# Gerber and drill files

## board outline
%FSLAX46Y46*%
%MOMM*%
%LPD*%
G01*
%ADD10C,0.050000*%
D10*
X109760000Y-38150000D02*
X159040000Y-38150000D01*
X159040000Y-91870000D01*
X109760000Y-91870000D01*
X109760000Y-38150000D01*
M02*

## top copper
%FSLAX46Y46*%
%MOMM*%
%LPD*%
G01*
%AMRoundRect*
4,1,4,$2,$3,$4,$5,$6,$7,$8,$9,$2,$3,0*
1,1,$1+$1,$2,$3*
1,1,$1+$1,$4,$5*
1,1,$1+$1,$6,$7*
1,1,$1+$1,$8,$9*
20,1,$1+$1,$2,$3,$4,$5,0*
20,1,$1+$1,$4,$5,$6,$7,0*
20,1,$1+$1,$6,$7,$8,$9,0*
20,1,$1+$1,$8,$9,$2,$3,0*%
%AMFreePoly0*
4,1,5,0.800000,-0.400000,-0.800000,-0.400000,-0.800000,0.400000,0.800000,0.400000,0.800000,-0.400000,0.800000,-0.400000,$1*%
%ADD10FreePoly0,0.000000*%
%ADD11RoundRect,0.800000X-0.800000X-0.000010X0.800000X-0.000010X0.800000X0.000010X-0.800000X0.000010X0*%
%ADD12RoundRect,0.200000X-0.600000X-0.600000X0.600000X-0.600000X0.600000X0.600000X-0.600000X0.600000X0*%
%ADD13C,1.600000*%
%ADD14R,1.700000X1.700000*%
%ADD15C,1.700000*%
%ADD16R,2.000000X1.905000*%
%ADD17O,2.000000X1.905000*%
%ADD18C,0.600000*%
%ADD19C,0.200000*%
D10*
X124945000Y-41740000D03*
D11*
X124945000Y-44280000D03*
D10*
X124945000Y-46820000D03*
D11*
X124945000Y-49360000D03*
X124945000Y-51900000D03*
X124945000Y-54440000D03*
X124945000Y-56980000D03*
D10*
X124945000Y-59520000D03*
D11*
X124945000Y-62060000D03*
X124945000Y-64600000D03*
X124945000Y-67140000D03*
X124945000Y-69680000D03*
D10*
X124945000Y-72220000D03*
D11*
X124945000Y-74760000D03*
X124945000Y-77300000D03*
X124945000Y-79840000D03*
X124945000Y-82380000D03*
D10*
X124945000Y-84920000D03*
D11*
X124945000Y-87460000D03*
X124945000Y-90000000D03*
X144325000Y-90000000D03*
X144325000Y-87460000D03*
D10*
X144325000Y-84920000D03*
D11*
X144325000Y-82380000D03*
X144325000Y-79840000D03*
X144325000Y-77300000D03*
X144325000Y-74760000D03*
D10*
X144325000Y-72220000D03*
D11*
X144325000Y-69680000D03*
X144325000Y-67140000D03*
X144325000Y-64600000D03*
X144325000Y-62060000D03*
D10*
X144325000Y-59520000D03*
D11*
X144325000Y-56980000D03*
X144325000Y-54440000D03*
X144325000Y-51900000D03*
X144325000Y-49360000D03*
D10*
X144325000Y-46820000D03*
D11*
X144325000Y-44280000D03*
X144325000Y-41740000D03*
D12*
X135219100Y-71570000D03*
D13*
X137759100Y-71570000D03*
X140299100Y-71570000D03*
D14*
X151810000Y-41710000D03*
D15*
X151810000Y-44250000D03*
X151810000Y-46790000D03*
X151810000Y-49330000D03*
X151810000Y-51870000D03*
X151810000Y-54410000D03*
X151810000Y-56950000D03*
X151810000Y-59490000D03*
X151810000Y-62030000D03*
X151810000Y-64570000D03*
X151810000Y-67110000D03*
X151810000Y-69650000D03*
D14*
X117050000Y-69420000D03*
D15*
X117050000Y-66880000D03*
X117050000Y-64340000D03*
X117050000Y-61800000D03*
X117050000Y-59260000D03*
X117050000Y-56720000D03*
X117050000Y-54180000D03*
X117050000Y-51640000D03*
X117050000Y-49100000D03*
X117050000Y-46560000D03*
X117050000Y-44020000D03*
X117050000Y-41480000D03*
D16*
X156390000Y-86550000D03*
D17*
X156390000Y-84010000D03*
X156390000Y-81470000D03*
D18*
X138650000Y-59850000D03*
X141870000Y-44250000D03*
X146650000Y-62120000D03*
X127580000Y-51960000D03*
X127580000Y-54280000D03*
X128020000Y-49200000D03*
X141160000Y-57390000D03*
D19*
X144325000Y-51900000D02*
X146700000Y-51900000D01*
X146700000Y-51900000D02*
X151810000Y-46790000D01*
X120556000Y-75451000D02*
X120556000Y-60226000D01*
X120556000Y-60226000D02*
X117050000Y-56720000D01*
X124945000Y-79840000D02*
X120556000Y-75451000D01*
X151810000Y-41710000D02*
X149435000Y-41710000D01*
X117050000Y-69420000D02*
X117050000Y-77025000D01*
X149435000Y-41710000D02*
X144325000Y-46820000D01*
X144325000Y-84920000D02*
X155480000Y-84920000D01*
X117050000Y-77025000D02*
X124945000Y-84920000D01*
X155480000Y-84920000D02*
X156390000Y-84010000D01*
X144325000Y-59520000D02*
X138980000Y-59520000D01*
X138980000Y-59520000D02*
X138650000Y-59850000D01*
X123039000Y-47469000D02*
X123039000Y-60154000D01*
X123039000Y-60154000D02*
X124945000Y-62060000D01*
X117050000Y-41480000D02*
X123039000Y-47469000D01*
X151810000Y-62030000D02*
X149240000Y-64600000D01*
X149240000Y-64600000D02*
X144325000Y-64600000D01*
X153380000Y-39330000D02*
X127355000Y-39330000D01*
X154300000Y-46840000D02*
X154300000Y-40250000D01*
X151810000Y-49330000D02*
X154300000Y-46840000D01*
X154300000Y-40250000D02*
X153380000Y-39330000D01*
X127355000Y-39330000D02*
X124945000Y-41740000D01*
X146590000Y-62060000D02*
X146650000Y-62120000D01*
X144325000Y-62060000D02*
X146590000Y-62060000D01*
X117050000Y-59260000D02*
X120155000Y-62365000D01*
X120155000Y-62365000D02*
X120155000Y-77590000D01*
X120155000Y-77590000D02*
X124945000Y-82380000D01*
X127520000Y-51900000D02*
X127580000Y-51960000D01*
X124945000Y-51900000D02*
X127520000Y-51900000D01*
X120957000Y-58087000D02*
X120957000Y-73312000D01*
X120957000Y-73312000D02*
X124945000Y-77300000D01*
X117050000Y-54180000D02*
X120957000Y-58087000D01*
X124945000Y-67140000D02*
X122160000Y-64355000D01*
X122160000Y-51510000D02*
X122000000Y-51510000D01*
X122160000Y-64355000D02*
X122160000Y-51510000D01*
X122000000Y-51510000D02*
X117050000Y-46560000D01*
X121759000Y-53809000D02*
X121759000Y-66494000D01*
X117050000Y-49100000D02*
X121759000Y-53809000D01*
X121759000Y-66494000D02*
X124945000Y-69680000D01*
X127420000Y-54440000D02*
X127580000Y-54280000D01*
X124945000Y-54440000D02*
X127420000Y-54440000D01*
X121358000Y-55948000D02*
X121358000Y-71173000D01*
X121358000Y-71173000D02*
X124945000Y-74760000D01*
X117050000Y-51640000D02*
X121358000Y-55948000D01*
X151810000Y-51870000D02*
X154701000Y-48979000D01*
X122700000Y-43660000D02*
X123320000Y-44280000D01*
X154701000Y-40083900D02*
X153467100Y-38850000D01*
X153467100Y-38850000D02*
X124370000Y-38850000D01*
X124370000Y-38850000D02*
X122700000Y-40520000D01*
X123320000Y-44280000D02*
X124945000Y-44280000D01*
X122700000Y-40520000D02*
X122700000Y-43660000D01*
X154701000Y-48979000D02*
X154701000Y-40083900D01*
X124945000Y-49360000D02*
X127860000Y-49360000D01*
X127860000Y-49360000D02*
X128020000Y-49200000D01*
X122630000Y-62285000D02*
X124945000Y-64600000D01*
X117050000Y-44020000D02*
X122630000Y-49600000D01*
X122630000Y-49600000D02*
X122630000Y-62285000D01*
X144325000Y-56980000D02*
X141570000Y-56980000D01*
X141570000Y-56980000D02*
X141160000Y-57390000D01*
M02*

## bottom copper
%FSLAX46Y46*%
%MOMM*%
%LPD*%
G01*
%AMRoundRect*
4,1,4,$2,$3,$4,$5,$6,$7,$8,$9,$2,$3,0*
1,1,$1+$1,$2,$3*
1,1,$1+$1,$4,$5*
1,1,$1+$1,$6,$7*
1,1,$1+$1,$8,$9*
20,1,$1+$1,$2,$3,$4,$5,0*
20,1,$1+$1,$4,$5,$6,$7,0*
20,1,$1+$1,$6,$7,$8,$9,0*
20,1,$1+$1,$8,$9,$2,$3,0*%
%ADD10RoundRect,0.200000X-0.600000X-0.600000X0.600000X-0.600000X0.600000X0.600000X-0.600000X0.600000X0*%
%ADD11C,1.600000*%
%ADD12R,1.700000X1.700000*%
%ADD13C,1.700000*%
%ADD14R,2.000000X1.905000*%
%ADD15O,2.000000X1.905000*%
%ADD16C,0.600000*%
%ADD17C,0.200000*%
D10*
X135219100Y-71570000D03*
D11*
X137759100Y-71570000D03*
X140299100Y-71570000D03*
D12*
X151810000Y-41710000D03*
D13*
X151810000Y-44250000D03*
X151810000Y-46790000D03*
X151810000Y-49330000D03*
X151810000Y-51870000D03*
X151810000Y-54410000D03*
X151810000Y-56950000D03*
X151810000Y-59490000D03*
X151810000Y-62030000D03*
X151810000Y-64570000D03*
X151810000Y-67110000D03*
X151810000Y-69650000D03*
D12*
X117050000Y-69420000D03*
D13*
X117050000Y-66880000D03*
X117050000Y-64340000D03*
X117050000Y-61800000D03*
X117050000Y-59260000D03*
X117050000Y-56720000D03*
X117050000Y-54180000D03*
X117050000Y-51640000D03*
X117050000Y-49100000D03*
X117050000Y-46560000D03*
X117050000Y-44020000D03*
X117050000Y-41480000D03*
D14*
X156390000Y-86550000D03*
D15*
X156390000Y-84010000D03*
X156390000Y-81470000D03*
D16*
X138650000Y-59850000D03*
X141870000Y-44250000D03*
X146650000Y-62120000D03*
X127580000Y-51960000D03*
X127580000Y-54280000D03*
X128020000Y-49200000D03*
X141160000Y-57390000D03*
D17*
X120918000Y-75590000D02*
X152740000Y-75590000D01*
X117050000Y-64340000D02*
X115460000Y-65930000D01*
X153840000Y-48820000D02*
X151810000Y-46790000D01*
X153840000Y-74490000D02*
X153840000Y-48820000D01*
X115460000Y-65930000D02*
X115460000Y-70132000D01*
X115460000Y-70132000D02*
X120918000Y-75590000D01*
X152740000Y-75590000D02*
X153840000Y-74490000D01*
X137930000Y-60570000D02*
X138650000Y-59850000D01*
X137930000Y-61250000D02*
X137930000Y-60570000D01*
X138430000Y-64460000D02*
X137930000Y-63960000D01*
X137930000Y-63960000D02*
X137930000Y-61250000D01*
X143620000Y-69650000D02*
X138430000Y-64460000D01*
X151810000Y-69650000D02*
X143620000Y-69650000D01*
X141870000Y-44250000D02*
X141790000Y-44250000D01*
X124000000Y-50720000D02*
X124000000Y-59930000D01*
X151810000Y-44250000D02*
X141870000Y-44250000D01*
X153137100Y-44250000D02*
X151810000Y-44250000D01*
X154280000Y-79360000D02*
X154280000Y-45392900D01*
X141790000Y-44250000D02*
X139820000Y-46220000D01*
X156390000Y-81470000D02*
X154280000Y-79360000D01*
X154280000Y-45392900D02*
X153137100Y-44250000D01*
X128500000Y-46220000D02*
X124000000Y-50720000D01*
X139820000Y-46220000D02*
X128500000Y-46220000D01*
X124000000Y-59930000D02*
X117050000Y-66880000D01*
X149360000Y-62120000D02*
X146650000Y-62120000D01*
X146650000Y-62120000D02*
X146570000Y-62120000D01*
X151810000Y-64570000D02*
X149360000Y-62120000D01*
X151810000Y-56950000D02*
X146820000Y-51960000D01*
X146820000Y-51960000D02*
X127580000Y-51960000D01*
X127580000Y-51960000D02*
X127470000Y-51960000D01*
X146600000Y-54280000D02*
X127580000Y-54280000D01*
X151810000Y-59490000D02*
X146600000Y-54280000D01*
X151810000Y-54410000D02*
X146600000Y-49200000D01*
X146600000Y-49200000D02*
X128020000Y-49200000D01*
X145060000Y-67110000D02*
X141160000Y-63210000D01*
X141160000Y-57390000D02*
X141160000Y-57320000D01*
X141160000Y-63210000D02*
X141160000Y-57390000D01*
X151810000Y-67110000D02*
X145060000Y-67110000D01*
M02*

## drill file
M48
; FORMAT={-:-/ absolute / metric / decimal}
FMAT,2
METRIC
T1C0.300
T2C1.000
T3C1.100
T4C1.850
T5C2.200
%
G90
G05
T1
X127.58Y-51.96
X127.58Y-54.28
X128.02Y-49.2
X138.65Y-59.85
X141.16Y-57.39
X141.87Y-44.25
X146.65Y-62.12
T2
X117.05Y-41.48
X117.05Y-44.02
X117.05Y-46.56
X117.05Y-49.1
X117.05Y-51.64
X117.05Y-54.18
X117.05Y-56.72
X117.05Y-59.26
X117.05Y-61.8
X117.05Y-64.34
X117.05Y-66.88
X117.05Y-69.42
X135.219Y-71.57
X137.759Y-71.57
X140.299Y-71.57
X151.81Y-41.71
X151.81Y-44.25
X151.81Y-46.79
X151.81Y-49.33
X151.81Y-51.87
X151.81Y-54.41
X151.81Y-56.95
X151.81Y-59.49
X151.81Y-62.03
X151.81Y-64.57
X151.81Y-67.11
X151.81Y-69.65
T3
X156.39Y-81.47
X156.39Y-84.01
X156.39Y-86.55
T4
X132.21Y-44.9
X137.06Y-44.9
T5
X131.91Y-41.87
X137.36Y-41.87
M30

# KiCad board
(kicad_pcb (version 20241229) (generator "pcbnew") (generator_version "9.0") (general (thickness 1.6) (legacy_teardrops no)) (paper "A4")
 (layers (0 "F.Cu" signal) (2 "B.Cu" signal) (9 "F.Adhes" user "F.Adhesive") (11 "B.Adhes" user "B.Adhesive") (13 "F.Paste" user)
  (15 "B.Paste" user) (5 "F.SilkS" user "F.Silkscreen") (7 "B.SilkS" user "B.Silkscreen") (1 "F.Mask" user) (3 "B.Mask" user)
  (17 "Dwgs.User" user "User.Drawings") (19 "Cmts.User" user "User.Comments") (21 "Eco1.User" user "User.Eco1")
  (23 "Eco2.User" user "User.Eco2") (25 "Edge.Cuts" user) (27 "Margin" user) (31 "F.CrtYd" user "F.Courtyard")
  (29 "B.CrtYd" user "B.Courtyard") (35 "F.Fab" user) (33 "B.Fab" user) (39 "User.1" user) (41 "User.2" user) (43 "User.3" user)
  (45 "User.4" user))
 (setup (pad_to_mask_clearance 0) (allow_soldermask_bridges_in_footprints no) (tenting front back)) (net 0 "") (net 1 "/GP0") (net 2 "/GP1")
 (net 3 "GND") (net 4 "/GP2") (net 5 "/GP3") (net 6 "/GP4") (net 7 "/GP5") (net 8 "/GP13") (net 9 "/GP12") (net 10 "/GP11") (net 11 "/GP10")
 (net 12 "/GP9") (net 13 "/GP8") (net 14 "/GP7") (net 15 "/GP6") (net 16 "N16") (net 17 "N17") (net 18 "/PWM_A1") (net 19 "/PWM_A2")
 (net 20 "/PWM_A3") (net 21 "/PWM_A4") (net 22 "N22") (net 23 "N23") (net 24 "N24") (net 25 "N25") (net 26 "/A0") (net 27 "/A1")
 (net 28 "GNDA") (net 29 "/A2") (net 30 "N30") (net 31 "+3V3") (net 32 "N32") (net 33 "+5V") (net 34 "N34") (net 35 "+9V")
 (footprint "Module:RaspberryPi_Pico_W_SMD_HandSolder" (layer "F.Cu") (at 134.635 65.87)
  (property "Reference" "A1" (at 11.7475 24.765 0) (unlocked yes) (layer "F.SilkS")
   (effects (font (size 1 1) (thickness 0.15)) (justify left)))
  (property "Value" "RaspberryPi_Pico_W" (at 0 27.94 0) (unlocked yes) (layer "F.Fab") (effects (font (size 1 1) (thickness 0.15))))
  (pad "" smd rect (at -8.89 -24.13) (size 3.8 2.2) (drill (offset -0.8 0)) (layers "F.Paste"))
  (pad "" smd rect (at -8.89 -21.59) (size 3.8 2.2) (drill (offset -0.8 0)) (layers "F.Paste"))
  (pad "" smd rect (at -8.89 -19.05) (size 3.8 2.2) (drill (offset -0.8 0)) (layers "F.Paste"))
  (pad "" smd rect (at -8.89 -16.51) (size 3.8 2.2) (drill (offset -0.8 0)) (layers "F.Paste"))
  (pad "" smd rect (at -8.89 -13.97) (size 3.8 2.2) (drill (offset -0.8 0)) (layers "F.Paste"))
  (pad "" smd rect (at -8.89 -11.43) (size 3.8 2.2) (drill (offset -0.8 0)) (layers "F.Paste"))
  (pad "" smd rect (at -8.89 -8.89) (size 3.8 2.2) (drill (offset -0.8 0)) (layers "F.Paste"))
  (pad "" smd rect (at -8.89 -6.35) (size 3.8 2.2) (drill (offset -0.8 0)) (layers "F.Paste"))
  (pad "" smd rect (at -8.89 -3.81) (size 3.8 2.2) (drill (offset -0.8 0)) (layers "F.Paste"))
  (pad "" smd rect (at -8.89 -1.27) (size 3.8 2.2) (drill (offset -0.8 0)) (layers "F.Paste"))
  (pad "" smd rect (at -8.89 1.27) (size 3.8 2.2) (drill (offset -0.8 0)) (layers "F.Paste"))
  (pad "" smd rect (at -8.89 3.81) (size 3.8 2.2) (drill (offset -0.8 0)) (layers "F.Paste"))
  (pad "" smd rect (at -8.89 6.35) (size 3.8 2.2) (drill (offset -0.8 0)) (layers "F.Paste"))
  (pad "" smd rect (at -8.89 8.89) (size 3.8 2.2) (drill (offset -0.8 0)) (layers "F.Paste"))
  (pad "" smd rect (at -8.89 11.43) (size 3.8 2.2) (drill (offset -0.8 0)) (layers "F.Paste"))
  (pad "" smd rect (at -8.89 13.97) (size 3.8 2.2) (drill (offset -0.8 0)) (layers "F.Paste"))
  (pad "" smd rect (at -8.89 16.51) (size 3.8 2.2) (drill (offset -0.8 0)) (layers "F.Paste"))
  (pad "" smd rect (at -8.89 19.05) (size 3.8 2.2) (drill (offset -0.8 0)) (layers "F.Paste"))
  (pad "" smd rect (at -8.89 21.59) (size 3.8 2.2) (drill (offset -0.8 0)) (layers "F.Paste"))
  (pad "" smd rect (at -8.89 24.13) (size 3.8 2.2) (drill (offset -0.8 0)) (layers "F.Paste"))
  (pad "" np_thru_hole circle (at -2.725 -24) (size 2.2 2.2) (drill 2.2) (layers "*.Mask"))
  (pad "" np_thru_hole circle (at -2.425 -20.97) (size 1.85 1.85) (drill 1.85) (layers "*.Mask"))
  (pad "" np_thru_hole circle (at 2.425 -20.97) (size 1.85 1.85) (drill 1.85) (layers "*.Mask"))
  (pad "" np_thru_hole circle (at 2.725 -24) (size 2.2 2.2) (drill 2.2) (layers "*.Mask"))
  (pad "" smd rect (at 8.89 -24.13) (size 3.8 2.2) (drill (offset 0.8 0)) (layers "F.Paste"))
  (pad "" smd rect (at 8.89 -21.59) (size 3.8 2.2) (drill (offset 0.8 0)) (layers "F.Paste"))
  (pad "" smd rect (at 8.89 -19.05) (size 3.8 2.2) (drill (offset 0.8 0)) (layers "F.Paste"))
  (pad "" smd rect (at 8.89 -16.51) (size 3.8 2.2) (drill (offset 0.8 0)) (layers "F.Paste"))
  (pad "" smd rect (at 8.89 -13.97) (size 3.8 2.2) (drill (offset 0.8 0)) (layers "F.Paste"))
  (pad "" smd rect (at 8.89 -11.43) (size 3.8 2.2) (drill (offset 0.8 0)) (layers "F.Paste"))
  (pad "" smd rect (at 8.89 -8.89) (size 3.8 2.2) (drill (offset 0.8 0)) (layers "F.Paste"))
  (pad "" smd rect (at 8.89 -6.35) (size 3.8 2.2) (drill (offset 0.8 0)) (layers "F.Paste"))
  (pad "" smd rect (at 8.89 -3.81) (size 3.8 2.2) (drill (offset 0.8 0)) (layers "F.Paste"))
  (pad "" smd rect (at 8.89 -1.27) (size 3.8 2.2) (drill (offset 0.8 0)) (layers "F.Paste"))
  (pad "" smd rect (at 8.89 1.27) (size 3.8 2.2) (drill (offset 0.8 0)) (layers "F.Paste"))
  (pad "" smd rect (at 8.89 3.81) (size 3.8 2.2) (drill (offset 0.8 0)) (layers "F.Paste"))
  (pad "" smd rect (at 8.89 6.35) (size 3.8 2.2) (drill (offset 0.8 0)) (layers "F.Paste"))
  (pad "" smd rect (at 8.89 8.89) (size 3.8 2.2) (drill (offset 0.8 0)) (layers "F.Paste"))
  (pad "" smd rect (at 8.89 11.43) (size 3.8 2.2) (drill (offset 0.8 0)) (layers "F.Paste"))
  (pad "" smd rect (at 8.89 13.97) (size 3.8 2.2) (drill (offset 0.8 0)) (layers "F.Paste"))
  (pad "" smd rect (at 8.89 16.51) (size 3.8 2.2) (drill (offset 0.8 0)) (layers "F.Paste"))
  (pad "" smd rect (at 8.89 19.05) (size 3.8 2.2) (drill (offset 0.8 0)) (layers "F.Paste"))
  (pad "" smd rect (at 8.89 21.59) (size 3.8 2.2) (drill (offset 0.8 0)) (layers "F.Paste"))
  (pad "" smd rect (at 8.89 24.13) (size 3.8 2.2) (drill (offset 0.8 0)) (layers "F.Paste"))
  (pad "1" smd custom (at -9.69 -24.13) (size 1.6 0.8) (layers "F.Cu" "F.Mask") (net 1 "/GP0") (options (clearance outline) (anchor rect))
   (primitives))
  (pad "2" smd roundrect (at -9.69 -21.59) (size 3.2 1.6) (layers "F.Cu" "F.Mask") (roundrect_rratio 0.5) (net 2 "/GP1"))
  (pad "3" smd custom (at -9.69 -19.05) (size 1.6 0.8) (layers "F.Cu" "F.Mask") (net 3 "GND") (options (clearance outline) (anchor rect))
   (primitives))
  (pad "4" smd roundrect (at -9.69 -16.51) (size 3.2 1.6) (layers "F.Cu" "F.Mask") (roundrect_rratio 0.5) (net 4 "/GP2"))
  (pad "5" smd roundrect (at -9.69 -13.97) (size 3.2 1.6) (layers "F.Cu" "F.Mask") (roundrect_rratio 0.5) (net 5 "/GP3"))
  (pad "6" smd roundrect (at -9.69 -11.43) (size 3.2 1.6) (layers "F.Cu" "F.Mask") (roundrect_rratio 0.5) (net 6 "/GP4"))
  (pad "7" smd roundrect (at -9.69 -8.89) (size 3.2 1.6) (layers "F.Cu" "F.Mask") (roundrect_rratio 0.5) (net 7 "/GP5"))
  (pad "8" smd custom (at -9.69 -6.35) (size 1.6 0.8) (layers "F.Cu" "F.Mask") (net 3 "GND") (options (clearance outline) (anchor rect))
   (primitives))
  (pad "9" smd roundrect (at -9.69 -3.81) (size 3.2 1.6) (layers "F.Cu" "F.Mask") (roundrect_rratio 0.5) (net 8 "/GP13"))
  (pad "10" smd roundrect (at -9.69 -1.27) (size 3.2 1.6) (layers "F.Cu" "F.Mask") (roundrect_rratio 0.5) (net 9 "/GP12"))
  (pad "11" smd roundrect (at -9.69 1.27) (size 3.2 1.6) (layers "F.Cu" "F.Mask") (roundrect_rratio 0.5) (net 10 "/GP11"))
  (pad "12" smd roundrect (at -9.69 3.81) (size 3.2 1.6) (layers "F.Cu" "F.Mask") (roundrect_rratio 0.5) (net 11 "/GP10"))
  (pad "13" smd custom (at -9.69 6.35) (size 1.6 0.8) (layers "F.Cu" "F.Mask") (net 3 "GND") (options (clearance outline) (anchor rect))
   (primitives))
  (pad "14" smd roundrect (at -9.69 8.89) (size 3.2 1.6) (layers "F.Cu" "F.Mask") (roundrect_rratio 0.5) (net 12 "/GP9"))
  (pad "15" smd roundrect (at -9.69 11.43) (size 3.2 1.6) (layers "F.Cu" "F.Mask") (roundrect_rratio 0.5) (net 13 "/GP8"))
  (pad "16" smd roundrect (at -9.69 13.97) (size 3.2 1.6) (layers "F.Cu" "F.Mask") (roundrect_rratio 0.5) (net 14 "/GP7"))
  (pad "17" smd roundrect (at -9.69 16.51) (size 3.2 1.6) (layers "F.Cu" "F.Mask") (roundrect_rratio 0.5) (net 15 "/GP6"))
  (pad "18" smd custom (at -9.69 19.05) (size 1.6 0.8) (layers "F.Cu" "F.Mask") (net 3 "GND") (options (clearance outline) (anchor rect))
   (primitives))
  (pad "19" smd roundrect (at -9.69 21.59) (size 3.2 1.6) (layers "F.Cu" "F.Mask") (roundrect_rratio 0.5) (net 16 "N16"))
  (pad "20" smd roundrect (at -9.69 24.13) (size 3.2 1.6) (layers "F.Cu" "F.Mask") (roundrect_rratio 0.5) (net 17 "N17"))
  (pad "21" smd roundrect (at 9.69 24.13) (size 3.2 1.6) (layers "F.Cu" "F.Mask") (roundrect_rratio 0.5) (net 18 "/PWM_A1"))
  (pad "22" smd roundrect (at 9.69 21.59) (size 3.2 1.6) (layers "F.Cu" "F.Mask") (roundrect_rratio 0.5) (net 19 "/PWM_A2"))
  (pad "23" smd custom (at 9.69 19.05) (size 1.6 0.8) (layers "F.Cu" "F.Mask") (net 3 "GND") (options (clearance outline) (anchor rect))
   (primitives))
  (pad "24" smd roundrect (at 9.69 16.51) (size 3.2 1.6) (layers "F.Cu" "F.Mask") (roundrect_rratio 0.5) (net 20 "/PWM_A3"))
  (pad "25" smd roundrect (at 9.69 13.97) (size 3.2 1.6) (layers "F.Cu" "F.Mask") (roundrect_rratio 0.5) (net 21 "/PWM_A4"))
  (pad "26" smd roundrect (at 9.69 11.43) (size 3.2 1.6) (layers "F.Cu" "F.Mask") (roundrect_rratio 0.5) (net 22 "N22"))
  (pad "27" smd roundrect (at 9.69 8.89) (size 3.2 1.6) (layers "F.Cu" "F.Mask") (roundrect_rratio 0.5) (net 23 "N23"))
  (pad "28" smd custom (at 9.69 6.35) (size 1.6 0.8) (layers "F.Cu" "F.Mask") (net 3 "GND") (options (clearance outline) (anchor rect))
   (primitives))
  (pad "29" smd roundrect (at 9.69 3.81) (size 3.2 1.6) (layers "F.Cu" "F.Mask") (roundrect_rratio 0.5) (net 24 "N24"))
  (pad "30" smd roundrect (at 9.69 1.27) (size 3.2 1.6) (layers "F.Cu" "F.Mask") (roundrect_rratio 0.5) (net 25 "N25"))
  (pad "31" smd roundrect (at 9.69 -1.27) (size 3.2 1.6) (layers "F.Cu" "F.Mask") (roundrect_rratio 0.5) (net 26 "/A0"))
  (pad "32" smd roundrect (at 9.69 -3.81) (size 3.2 1.6) (layers "F.Cu" "F.Mask") (roundrect_rratio 0.5) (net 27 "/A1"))
  (pad "33" smd custom (at 9.69 -6.35) (size 1.6 0.8) (layers "F.Cu" "F.Mask") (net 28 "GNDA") (options (clearance outline) (anchor rect))
   (primitives))
  (pad "34" smd roundrect (at 9.69 -8.89) (size 3.2 1.6) (layers "F.Cu" "F.Mask") (roundrect_rratio 0.5) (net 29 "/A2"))
  (pad "35" smd roundrect (at 9.69 -11.43) (size 3.2 1.6) (layers "F.Cu" "F.Mask") (roundrect_rratio 0.5) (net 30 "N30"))
  (pad "36" smd roundrect (at 9.69 -13.97) (size 3.2 1.6) (layers "F.Cu" "F.Mask") (roundrect_rratio 0.5) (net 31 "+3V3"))
  (pad "37" smd roundrect (at 9.69 -16.51) (size 3.2 1.6) (layers "F.Cu" "F.Mask") (roundrect_rratio 0.5) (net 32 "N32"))
  (pad "38" smd custom (at 9.69 -19.05) (size 1.6 0.8) (layers "F.Cu" "F.Mask") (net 3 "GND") (options (clearance outline) (anchor rect))
   (primitives))
  (pad "39" smd roundrect (at 9.69 -21.59) (size 3.2 1.6) (layers "F.Cu" "F.Mask") (roundrect_rratio 0.5) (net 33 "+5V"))
  (pad "40" smd roundrect (at 9.69 -24.13) (size 3.2 1.6) (layers "F.Cu" "F.Mask") (roundrect_rratio 0.5) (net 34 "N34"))
  (pad "D1" thru_hole roundrect (at 0.5841 5.7) (size 1.6 1.6) (drill 1) (layers "*.Cu" "*.Mask") (remove_unused_layers no)
   (roundrect_rratio 0.125))
  (pad "D2" thru_hole circle (at 3.1241 5.7) (size 1.6 1.6) (drill 1) (layers "*.Cu" "*.Mask") (remove_unused_layers no))
  (pad "D3" thru_hole circle (at 5.6641 5.7) (size 1.6 1.6) (drill 1) (layers "*.Cu" "*.Mask") (remove_unused_layers no))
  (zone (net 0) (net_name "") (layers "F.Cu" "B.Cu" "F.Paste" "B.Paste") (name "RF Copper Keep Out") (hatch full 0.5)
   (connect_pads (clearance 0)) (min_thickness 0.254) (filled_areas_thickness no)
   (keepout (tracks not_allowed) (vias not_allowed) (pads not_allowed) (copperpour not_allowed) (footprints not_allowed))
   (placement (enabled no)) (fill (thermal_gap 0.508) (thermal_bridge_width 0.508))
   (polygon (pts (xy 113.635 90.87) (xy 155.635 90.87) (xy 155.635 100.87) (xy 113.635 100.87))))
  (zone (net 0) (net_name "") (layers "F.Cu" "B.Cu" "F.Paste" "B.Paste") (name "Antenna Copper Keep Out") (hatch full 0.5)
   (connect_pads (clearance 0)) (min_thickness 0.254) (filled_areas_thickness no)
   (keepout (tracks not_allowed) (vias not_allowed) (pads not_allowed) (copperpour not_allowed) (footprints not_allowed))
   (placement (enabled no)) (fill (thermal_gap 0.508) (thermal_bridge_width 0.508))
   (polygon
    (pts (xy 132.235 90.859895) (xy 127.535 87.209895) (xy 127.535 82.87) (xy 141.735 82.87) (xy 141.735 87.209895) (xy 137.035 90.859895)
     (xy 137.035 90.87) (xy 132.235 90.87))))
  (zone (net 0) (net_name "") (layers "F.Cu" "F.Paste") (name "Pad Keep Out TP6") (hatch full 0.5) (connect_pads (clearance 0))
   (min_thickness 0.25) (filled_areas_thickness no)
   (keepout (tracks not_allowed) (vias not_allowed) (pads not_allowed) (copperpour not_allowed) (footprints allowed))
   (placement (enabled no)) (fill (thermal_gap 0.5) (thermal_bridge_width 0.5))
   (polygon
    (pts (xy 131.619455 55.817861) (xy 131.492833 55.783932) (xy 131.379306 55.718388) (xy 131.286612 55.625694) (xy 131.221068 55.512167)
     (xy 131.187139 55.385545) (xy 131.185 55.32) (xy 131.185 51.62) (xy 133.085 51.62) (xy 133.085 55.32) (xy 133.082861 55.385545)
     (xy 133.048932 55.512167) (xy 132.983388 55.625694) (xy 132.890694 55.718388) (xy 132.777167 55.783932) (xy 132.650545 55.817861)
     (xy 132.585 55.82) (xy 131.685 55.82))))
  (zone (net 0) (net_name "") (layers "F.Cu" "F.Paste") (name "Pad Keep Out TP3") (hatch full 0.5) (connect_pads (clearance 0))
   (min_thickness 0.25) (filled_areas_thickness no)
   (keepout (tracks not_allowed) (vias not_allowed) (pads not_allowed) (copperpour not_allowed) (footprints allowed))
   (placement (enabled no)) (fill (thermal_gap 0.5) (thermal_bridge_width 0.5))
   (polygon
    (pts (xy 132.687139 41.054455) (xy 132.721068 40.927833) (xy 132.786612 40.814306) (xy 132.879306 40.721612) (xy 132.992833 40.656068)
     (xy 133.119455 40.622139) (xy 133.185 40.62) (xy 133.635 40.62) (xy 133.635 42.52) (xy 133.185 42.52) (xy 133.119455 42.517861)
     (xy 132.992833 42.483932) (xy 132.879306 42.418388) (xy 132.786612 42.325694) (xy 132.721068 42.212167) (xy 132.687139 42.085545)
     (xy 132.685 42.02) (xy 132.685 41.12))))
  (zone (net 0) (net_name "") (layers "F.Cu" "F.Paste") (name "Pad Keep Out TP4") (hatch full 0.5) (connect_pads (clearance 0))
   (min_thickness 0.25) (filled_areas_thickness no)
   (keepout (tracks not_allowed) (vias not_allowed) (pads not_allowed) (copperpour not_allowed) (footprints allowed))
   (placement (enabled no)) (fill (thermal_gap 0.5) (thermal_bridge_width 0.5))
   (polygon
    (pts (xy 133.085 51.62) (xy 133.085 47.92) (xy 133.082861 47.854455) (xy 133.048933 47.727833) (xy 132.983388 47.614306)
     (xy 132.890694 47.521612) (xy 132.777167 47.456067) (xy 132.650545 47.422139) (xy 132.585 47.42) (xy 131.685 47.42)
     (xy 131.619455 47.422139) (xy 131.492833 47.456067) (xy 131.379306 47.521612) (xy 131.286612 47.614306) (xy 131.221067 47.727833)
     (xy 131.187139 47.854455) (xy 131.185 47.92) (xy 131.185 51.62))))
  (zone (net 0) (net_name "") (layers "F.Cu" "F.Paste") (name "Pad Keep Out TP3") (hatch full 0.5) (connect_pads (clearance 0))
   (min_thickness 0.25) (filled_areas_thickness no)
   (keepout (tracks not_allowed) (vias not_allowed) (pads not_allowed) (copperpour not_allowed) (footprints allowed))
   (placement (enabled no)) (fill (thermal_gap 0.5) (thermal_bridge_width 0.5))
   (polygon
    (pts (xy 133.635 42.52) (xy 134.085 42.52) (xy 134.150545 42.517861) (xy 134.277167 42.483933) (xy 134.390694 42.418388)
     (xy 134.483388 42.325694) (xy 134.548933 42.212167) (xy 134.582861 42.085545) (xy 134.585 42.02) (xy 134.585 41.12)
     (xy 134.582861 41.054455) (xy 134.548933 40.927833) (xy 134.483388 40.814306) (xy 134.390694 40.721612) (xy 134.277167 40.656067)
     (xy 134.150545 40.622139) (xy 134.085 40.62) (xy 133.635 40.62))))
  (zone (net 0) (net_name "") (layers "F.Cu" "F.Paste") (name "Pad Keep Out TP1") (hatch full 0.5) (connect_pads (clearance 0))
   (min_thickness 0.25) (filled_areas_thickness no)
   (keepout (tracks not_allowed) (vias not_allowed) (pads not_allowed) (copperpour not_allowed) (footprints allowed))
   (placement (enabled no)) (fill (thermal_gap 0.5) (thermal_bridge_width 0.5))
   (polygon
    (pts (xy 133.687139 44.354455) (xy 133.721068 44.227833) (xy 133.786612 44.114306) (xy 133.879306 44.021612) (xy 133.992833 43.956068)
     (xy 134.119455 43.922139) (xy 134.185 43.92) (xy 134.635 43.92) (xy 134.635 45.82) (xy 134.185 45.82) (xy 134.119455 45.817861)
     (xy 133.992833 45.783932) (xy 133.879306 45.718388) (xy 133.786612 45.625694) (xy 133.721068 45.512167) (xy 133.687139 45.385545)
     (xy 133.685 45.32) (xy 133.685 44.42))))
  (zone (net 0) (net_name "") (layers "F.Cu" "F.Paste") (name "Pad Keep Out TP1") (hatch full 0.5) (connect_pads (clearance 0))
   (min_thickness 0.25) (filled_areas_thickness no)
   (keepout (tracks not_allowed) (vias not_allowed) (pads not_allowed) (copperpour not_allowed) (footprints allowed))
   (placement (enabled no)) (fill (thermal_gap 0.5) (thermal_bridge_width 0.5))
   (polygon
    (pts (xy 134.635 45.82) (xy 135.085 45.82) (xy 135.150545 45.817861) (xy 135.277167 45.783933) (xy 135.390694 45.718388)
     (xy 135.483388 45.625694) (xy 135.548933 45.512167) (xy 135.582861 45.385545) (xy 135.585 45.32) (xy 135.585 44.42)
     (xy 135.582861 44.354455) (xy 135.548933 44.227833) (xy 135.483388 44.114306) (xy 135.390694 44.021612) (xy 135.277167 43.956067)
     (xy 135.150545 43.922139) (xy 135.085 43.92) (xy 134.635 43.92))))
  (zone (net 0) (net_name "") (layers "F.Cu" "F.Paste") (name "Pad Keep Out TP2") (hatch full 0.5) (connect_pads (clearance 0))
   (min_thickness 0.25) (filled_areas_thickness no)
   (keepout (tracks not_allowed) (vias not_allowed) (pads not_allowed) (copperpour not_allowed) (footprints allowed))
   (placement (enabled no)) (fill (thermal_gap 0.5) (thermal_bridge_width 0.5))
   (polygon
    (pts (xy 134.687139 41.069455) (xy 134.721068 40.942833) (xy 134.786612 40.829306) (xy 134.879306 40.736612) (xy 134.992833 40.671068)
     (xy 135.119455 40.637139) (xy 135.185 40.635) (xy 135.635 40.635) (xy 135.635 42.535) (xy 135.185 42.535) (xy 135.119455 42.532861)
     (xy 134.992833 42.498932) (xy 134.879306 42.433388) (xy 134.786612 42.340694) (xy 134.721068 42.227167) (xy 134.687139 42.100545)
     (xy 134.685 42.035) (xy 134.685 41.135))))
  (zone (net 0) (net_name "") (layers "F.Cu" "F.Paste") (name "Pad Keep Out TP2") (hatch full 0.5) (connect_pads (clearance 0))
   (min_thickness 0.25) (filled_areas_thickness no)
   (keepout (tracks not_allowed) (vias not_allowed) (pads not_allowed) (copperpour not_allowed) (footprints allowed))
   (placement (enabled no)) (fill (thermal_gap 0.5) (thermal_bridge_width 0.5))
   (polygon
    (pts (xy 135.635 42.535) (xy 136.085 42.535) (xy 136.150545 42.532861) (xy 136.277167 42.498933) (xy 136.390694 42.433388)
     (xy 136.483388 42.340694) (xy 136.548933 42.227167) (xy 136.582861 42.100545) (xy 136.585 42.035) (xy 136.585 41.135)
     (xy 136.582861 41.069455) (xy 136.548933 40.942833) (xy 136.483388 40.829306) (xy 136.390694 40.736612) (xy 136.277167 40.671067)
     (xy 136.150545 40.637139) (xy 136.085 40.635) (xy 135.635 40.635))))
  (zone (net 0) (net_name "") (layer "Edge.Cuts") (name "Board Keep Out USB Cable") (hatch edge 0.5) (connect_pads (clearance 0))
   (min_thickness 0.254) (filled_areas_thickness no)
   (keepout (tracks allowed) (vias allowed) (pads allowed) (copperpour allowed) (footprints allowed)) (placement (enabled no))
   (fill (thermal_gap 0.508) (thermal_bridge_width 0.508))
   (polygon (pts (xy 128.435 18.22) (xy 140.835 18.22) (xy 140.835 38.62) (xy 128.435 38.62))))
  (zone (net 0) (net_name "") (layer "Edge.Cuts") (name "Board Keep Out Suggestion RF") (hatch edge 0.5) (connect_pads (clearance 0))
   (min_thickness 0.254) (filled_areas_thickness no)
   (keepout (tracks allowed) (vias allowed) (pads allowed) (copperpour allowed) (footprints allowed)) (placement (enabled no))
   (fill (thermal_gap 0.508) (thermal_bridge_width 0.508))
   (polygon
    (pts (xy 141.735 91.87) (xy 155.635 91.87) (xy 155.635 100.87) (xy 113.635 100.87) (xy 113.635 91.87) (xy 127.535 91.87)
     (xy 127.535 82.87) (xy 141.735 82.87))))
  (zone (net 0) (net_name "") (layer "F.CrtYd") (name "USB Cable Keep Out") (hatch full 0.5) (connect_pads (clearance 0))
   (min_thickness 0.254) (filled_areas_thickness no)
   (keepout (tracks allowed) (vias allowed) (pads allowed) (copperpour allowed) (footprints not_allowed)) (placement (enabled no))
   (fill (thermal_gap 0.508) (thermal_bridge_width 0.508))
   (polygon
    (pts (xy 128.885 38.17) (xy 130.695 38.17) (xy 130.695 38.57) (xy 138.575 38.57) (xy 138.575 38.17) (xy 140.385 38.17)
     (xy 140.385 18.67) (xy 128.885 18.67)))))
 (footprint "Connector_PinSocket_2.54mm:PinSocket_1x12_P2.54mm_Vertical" (layer "F.Cu") (at 151.81 41.71)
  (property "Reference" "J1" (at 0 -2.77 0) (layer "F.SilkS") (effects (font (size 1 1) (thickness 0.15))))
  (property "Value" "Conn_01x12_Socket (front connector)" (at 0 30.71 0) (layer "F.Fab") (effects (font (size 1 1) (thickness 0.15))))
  (pad "1" thru_hole rect (at 0 0) (size 1.7 1.7) (drill 1) (layers "*.Cu" "*.Mask") (remove_unused_layers no) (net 3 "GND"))
  (pad "2" thru_hole circle (at 0 2.54) (size 1.7 1.7) (drill 1) (layers "*.Cu" "*.Mask") (remove_unused_layers no) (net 33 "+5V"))
  (pad "3" thru_hole circle (at 0 5.08) (size 1.7 1.7) (drill 1) (layers "*.Cu" "*.Mask") (remove_unused_layers no) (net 31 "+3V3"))
  (pad "4" thru_hole circle (at 0 7.62) (size 1.7 1.7) (drill 1) (layers "*.Cu" "*.Mask") (remove_unused_layers no) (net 1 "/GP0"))
  (pad "5" thru_hole circle (at 0 10.16) (size 1.7 1.7) (drill 1) (layers "*.Cu" "*.Mask") (remove_unused_layers no) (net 2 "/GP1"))
  (pad "6" thru_hole circle (at 0 12.7) (size 1.7 1.7) (drill 1) (layers "*.Cu" "*.Mask") (remove_unused_layers no) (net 4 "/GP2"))
  (pad "7" thru_hole circle (at 0 15.24) (size 1.7 1.7) (drill 1) (layers "*.Cu" "*.Mask") (remove_unused_layers no) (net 5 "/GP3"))
  (pad "8" thru_hole circle (at 0 17.78) (size 1.7 1.7) (drill 1) (layers "*.Cu" "*.Mask") (remove_unused_layers no) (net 6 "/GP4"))
  (pad "9" thru_hole circle (at 0 20.32) (size 1.7 1.7) (drill 1) (layers "*.Cu" "*.Mask") (remove_unused_layers no) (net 26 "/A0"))
  (pad "10" thru_hole circle (at 0 22.86) (size 1.7 1.7) (drill 1) (layers "*.Cu" "*.Mask") (remove_unused_layers no) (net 27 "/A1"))
  (pad "11" thru_hole circle (at 0 25.4) (size 1.7 1.7) (drill 1) (layers "*.Cu" "*.Mask") (remove_unused_layers no) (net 29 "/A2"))
  (pad "12" thru_hole circle (at 0 27.94) (size 1.7 1.7) (drill 1) (layers "*.Cu" "*.Mask") (remove_unused_layers no) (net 28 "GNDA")))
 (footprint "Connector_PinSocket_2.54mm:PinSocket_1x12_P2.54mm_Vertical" (layer "F.Cu") (at 117.05 69.42 180)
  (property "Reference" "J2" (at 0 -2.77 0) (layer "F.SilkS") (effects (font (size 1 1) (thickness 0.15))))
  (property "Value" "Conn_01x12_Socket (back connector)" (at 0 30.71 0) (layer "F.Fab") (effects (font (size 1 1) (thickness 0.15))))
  (pad "1" thru_hole rect (at 0 0 180) (size 1.7 1.7) (drill 1) (layers "*.Cu" "*.Mask") (remove_unused_layers no) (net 3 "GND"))
  (pad "2" thru_hole circle (at 0 2.54 180) (size 1.7 1.7) (drill 1) (layers "*.Cu" "*.Mask") (remove_unused_layers no) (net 33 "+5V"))
  (pad "3" thru_hole circle (at 0 5.08 180) (size 1.7 1.7) (drill 1) (layers "*.Cu" "*.Mask") (remove_unused_layers no) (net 31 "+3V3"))
  (pad "4" thru_hole circle (at 0 7.62 180) (size 1.7 1.7) (drill 1) (layers "*.Cu" "*.Mask") (remove_unused_layers no) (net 7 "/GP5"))
  (pad "5" thru_hole circle (at 0 10.16 180) (size 1.7 1.7) (drill 1) (layers "*.Cu" "*.Mask") (remove_unused_layers no) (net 15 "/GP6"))
  (pad "6" thru_hole circle (at 0 12.7 180) (size 1.7 1.7) (drill 1) (layers "*.Cu" "*.Mask") (remove_unused_layers no) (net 14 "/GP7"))
  (pad "7" thru_hole circle (at 0 15.24 180) (size 1.7 1.7) (drill 1) (layers "*.Cu" "*.Mask") (remove_unused_layers no) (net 13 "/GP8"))
  (pad "8" thru_hole circle (at 0 17.78 180) (size 1.7 1.7) (drill 1) (layers "*.Cu" "*.Mask") (remove_unused_layers no) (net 12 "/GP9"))
  (pad "9" thru_hole circle (at 0 20.32 180) (size 1.7 1.7) (drill 1) (layers "*.Cu" "*.Mask") (remove_unused_layers no) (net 11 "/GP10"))
  (pad "10" thru_hole circle (at 0 22.86 180) (size 1.7 1.7) (drill 1) (layers "*.Cu" "*.Mask") (remove_unused_layers no) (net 10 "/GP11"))
  (pad "11" thru_hole circle (at 0 25.4 180) (size 1.7 1.7) (drill 1) (layers "*.Cu" "*.Mask") (remove_unused_layers no) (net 9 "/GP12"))
  (pad "12" thru_hole circle (at 0 27.94 180) (size 1.7 1.7) (drill 1) (layers "*.Cu" "*.Mask") (remove_unused_layers no) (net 8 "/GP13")))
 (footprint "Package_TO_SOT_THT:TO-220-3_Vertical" (layer "F.Cu") (at 156.39 86.55 90)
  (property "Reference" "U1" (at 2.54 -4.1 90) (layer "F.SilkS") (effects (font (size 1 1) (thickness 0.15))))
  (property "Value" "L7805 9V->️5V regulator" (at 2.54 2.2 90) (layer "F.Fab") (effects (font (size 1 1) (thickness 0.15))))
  (pad "1" thru_hole rect (at 0 0 90) (size 1.905 2) (drill 1.1) (layers "*.Cu" "*.Mask") (remove_unused_layers no) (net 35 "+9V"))
  (pad "2" thru_hole oval (at 2.54 0 90) (size 1.905 2) (drill 1.1) (layers "*.Cu" "*.Mask") (remove_unused_layers no) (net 3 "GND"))
  (pad "3" thru_hole oval (at 5.08 0 90) (size 1.905 2) (drill 1.1) (layers "*.Cu" "*.Mask") (remove_unused_layers no) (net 33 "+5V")))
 (gr_rect (start 109.76 38.15) (end 159.04 91.87) (stroke (width 0.05) (type default)) (fill no) (layer "Edge.Cuts"))
 (segment (start 144.325 51.9) (end 146.7 51.9) (width 0.2) (layer "F.Cu") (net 31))
 (segment (start 146.7 51.9) (end 151.81 46.79) (width 0.2) (layer "F.Cu") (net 31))
 (segment (start 120.918 75.59) (end 152.74 75.59) (width 0.2) (layer "B.Cu") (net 31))
 (segment (start 117.05 64.34) (end 115.46 65.93) (width 0.2) (layer "B.Cu") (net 31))
 (segment (start 153.84 48.82) (end 151.81 46.79) (width 0.2) (layer "B.Cu") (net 31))
 (segment (start 153.84 74.49) (end 153.84 48.82) (width 0.2) (layer "B.Cu") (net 31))
 (segment (start 115.46 65.93) (end 115.46 70.132) (width 0.2) (layer "B.Cu") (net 31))
 (segment (start 115.46 70.132) (end 120.918 75.59) (width 0.2) (layer "B.Cu") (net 31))
 (segment (start 152.74 75.59) (end 153.84 74.49) (width 0.2) (layer "B.Cu") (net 31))
 (segment (start 120.556 75.451) (end 120.556 60.226) (width 0.2) (layer "F.Cu") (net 14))
 (segment (start 120.556 60.226) (end 117.05 56.72) (width 0.2) (layer "F.Cu") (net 14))
 (segment (start 124.945 79.84) (end 120.556 75.451) (width 0.2) (layer "F.Cu") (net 14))
 (segment (start 151.81 41.71) (end 149.435 41.71) (width 0.2) (layer "F.Cu") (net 3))
 (segment (start 117.05 69.42) (end 117.05 77.025) (width 0.2) (layer "F.Cu") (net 3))
 (segment (start 149.435 41.71) (end 144.325 46.82) (width 0.2) (layer "F.Cu") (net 3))
 (segment (start 144.325 84.92) (end 155.48 84.92) (width 0.2) (layer "F.Cu") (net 3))
 (segment (start 117.05 77.025) (end 124.945 84.92) (width 0.2) (layer "F.Cu") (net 3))
 (segment (start 155.48 84.92) (end 156.39 84.01) (width 0.2) (layer "F.Cu") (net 3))
 (segment (start 144.325 59.52) (end 138.98 59.52) (width 0.2) (layer "F.Cu") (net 28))
 (segment (start 138.98 59.52) (end 138.65 59.85) (width 0.2) (layer "F.Cu") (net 28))
 (via (at 138.65 59.85) (size 0.6) (drill 0.3) (layers "F.Cu" "B.Cu") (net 28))
 (segment (start 137.93 60.57) (end 138.65 59.85) (width 0.2) (layer "B.Cu") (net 28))
 (segment (start 137.93 61.25) (end 137.93 60.57) (width 0.2) (layer "B.Cu") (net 28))
 (segment (start 138.43 64.46) (end 137.93 63.96) (width 0.2) (layer "B.Cu") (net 28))
 (segment (start 137.93 63.96) (end 137.93 61.25) (width 0.2) (layer "B.Cu") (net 28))
 (segment (start 143.62 69.65) (end 138.43 64.46) (width 0.2) (layer "B.Cu") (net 28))
 (segment (start 151.81 69.65) (end 143.62 69.65) (width 0.2) (layer "B.Cu") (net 28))
 (segment (start 123.039 47.469) (end 123.039 60.154) (width 0.2) (layer "F.Cu") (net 8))
 (segment (start 123.039 60.154) (end 124.945 62.06) (width 0.2) (layer "F.Cu") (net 8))
 (segment (start 117.05 41.48) (end 123.039 47.469) (width 0.2) (layer "F.Cu") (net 8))
 (segment (start 151.81 62.03) (end 149.24 64.6) (width 0.2) (layer "F.Cu") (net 26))
 (segment (start 149.24 64.6) (end 144.325 64.6) (width 0.2) (layer "F.Cu") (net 26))
 (via (at 141.87 44.25) (size 0.6) (drill 0.3) (layers "F.Cu" "B.Cu") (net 33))
 (segment (start 141.87 44.25) (end 141.79 44.25) (width 0.2) (layer "B.Cu") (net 33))
 (segment (start 124 50.72) (end 124 59.93) (width 0.2) (layer "B.Cu") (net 33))
 (segment (start 151.81 44.25) (end 141.87 44.25) (width 0.2) (layer "B.Cu") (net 33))
 (segment (start 153.1371 44.25) (end 151.81 44.25) (width 0.2) (layer "B.Cu") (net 33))
 (segment (start 154.28 79.36) (end 154.28 45.3929) (width 0.2) (layer "B.Cu") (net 33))
 (segment (start 141.79 44.25) (end 139.82 46.22) (width 0.2) (layer "B.Cu") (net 33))
 (segment (start 156.39 81.47) (end 154.28 79.36) (width 0.2) (layer "B.Cu") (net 33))
 (segment (start 154.28 45.3929) (end 153.1371 44.25) (width 0.2) (layer "B.Cu") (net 33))
 (segment (start 128.5 46.22) (end 124 50.72) (width 0.2) (layer "B.Cu") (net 33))
 (segment (start 139.82 46.22) (end 128.5 46.22) (width 0.2) (layer "B.Cu") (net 33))
 (segment (start 124 59.93) (end 117.05 66.88) (width 0.2) (layer "B.Cu") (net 33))
 (segment (start 153.38 39.33) (end 127.355 39.33) (width 0.2) (layer "F.Cu") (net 1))
 (segment (start 154.3 46.84) (end 154.3 40.25) (width 0.2) (layer "F.Cu") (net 1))
 (segment (start 151.81 49.33) (end 154.3 46.84) (width 0.2) (layer "F.Cu") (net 1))
 (segment (start 154.3 40.25) (end 153.38 39.33) (width 0.2) (layer "F.Cu") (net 1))
 (segment (start 127.355 39.33) (end 124.945 41.74) (width 0.2) (layer "F.Cu") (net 1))
 (segment (start 146.59 62.06) (end 146.65 62.12) (width 0.2) (layer "F.Cu") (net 27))
 (segment (start 144.325 62.06) (end 146.59 62.06) (width 0.2) (layer "F.Cu") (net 27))
 (via (at 146.65 62.12) (size 0.6) (drill 0.3) (layers "F.Cu" "B.Cu") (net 27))
 (segment (start 149.36 62.12) (end 146.65 62.12) (width 0.2) (layer "B.Cu") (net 27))
 (segment (start 146.65 62.12) (end 146.57 62.12) (width 0.2) (layer "B.Cu") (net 27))
 (segment (start 151.81 64.57) (end 149.36 62.12) (width 0.2) (layer "B.Cu") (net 27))
 (segment (start 117.05 59.26) (end 120.155 62.365) (width 0.2) (layer "F.Cu") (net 15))
 (segment (start 120.155 62.365) (end 120.155 77.59) (width 0.2) (layer "F.Cu") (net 15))
 (segment (start 120.155 77.59) (end 124.945 82.38) (width 0.2) (layer "F.Cu") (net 15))
 (segment (start 127.52 51.9) (end 127.58 51.96) (width 0.2) (layer "F.Cu") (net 5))
 (segment (start 124.945 51.9) (end 127.52 51.9) (width 0.2) (layer "F.Cu") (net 5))
 (via (at 127.58 51.96) (size 0.6) (drill 0.3) (layers "F.Cu" "B.Cu") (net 5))
 (segment (start 151.81 56.95) (end 146.82 51.96) (width 0.2) (layer "B.Cu") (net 5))
 (segment (start 146.82 51.96) (end 127.58 51.96) (width 0.2) (layer "B.Cu") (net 5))
 (segment (start 127.58 51.96) (end 127.47 51.96) (width 0.2) (layer "B.Cu") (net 5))
 (segment (start 120.957 58.087) (end 120.957 73.312) (width 0.2) (layer "F.Cu") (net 13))
 (segment (start 120.957 73.312) (end 124.945 77.3) (width 0.2) (layer "F.Cu") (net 13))
 (segment (start 117.05 54.18) (end 120.957 58.087) (width 0.2) (layer "F.Cu") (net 13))
 (segment (start 124.945 67.14) (end 122.16 64.355) (width 0.2) (layer "F.Cu") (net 10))
 (segment (start 122.16 51.51) (end 122 51.51) (width 0.2) (layer "F.Cu") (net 10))
 (segment (start 122.16 64.355) (end 122.16 51.51) (width 0.2) (layer "F.Cu") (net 10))
 (segment (start 122 51.51) (end 117.05 46.56) (width 0.2) (layer "F.Cu") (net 10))
 (segment (start 121.759 53.809) (end 121.759 66.494) (width 0.2) (layer "F.Cu") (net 11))
 (segment (start 117.05 49.1) (end 121.759 53.809) (width 0.2) (layer "F.Cu") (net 11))
 (segment (start 121.759 66.494) (end 124.945 69.68) (width 0.2) (layer "F.Cu") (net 11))
 (segment (start 127.42 54.44) (end 127.58 54.28) (width 0.2) (layer "F.Cu") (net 6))
 (segment (start 124.945 54.44) (end 127.42 54.44) (width 0.2) (layer "F.Cu") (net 6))
 (via (at 127.58 54.28) (size 0.6) (drill 0.3) (layers "F.Cu" "B.Cu") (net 6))
 (segment (start 146.6 54.28) (end 127.58 54.28) (width 0.2) (layer "B.Cu") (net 6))
 (segment (start 151.81 59.49) (end 146.6 54.28) (width 0.2) (layer "B.Cu") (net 6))
 (segment (start 121.358 55.948) (end 121.358 71.173) (width 0.2) (layer "F.Cu") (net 12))
 (segment (start 121.358 71.173) (end 124.945 74.76) (width 0.2) (layer "F.Cu") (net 12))
 (segment (start 117.05 51.64) (end 121.358 55.948) (width 0.2) (layer "F.Cu") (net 12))
 (segment (start 151.81 51.87) (end 154.701 48.979) (width 0.2) (layer "F.Cu") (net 2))
 (segment (start 122.7 43.66) (end 123.32 44.28) (width 0.2) (layer "F.Cu") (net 2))
 (segment (start 154.701 40.0839) (end 153.4671 38.85) (width 0.2) (layer "F.Cu") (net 2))
 (segment (start 153.4671 38.85) (end 124.37 38.85) (width 0.2) (layer "F.Cu") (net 2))
 (segment (start 124.37 38.85) (end 122.7 40.52) (width 0.2) (layer "F.Cu") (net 2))
 (segment (start 123.32 44.28) (end 124.945 44.28) (width 0.2) (layer "F.Cu") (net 2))
 (segment (start 122.7 40.52) (end 122.7 43.66) (width 0.2) (layer "F.Cu") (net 2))
 (segment (start 154.701 48.979) (end 154.701 40.0839) (width 0.2) (layer "F.Cu") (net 2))
 (segment (start 124.945 49.36) (end 127.86 49.36) (width 0.2) (layer "F.Cu") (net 4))
 (segment (start 127.86 49.36) (end 128.02 49.2) (width 0.2) (layer "F.Cu") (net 4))
 (via (at 128.02 49.2) (size 0.6) (drill 0.3) (layers "F.Cu" "B.Cu") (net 4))
 (segment (start 151.81 54.41) (end 146.6 49.2) (width 0.2) (layer "B.Cu") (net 4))
 (segment (start 146.6 49.2) (end 128.02 49.2) (width 0.2) (layer "B.Cu") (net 4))
 (segment (start 122.63 62.285) (end 124.945 64.6) (width 0.2) (layer "F.Cu") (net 9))
 (segment (start 117.05 44.02) (end 122.63 49.6) (width 0.2) (layer "F.Cu") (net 9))
 (segment (start 122.63 49.6) (end 122.63 62.285) (width 0.2) (layer "F.Cu") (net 9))
 (segment (start 144.325 56.98) (end 141.57 56.98) (width 0.2) (layer "F.Cu") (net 29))
 (segment (start 141.57 56.98) (end 141.16 57.39) (width 0.2) (layer "F.Cu") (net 29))
 (via (at 141.16 57.39) (size 0.6) (drill 0.3) (layers "F.Cu" "B.Cu") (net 29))
 (segment (start 145.06 67.11) (end 141.16 63.21) (width 0.2) (layer "B.Cu") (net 29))
 (segment (start 141.16 57.39) (end 141.16 57.32) (width 0.2) (layer "B.Cu") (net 29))
 (segment (start 141.16 63.21) (end 141.16 57.39) (width 0.2) (layer "B.Cu") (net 29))
 (segment (start 151.81 67.11) (end 145.06 67.11) (width 0.2) (layer "B.Cu") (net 29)))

